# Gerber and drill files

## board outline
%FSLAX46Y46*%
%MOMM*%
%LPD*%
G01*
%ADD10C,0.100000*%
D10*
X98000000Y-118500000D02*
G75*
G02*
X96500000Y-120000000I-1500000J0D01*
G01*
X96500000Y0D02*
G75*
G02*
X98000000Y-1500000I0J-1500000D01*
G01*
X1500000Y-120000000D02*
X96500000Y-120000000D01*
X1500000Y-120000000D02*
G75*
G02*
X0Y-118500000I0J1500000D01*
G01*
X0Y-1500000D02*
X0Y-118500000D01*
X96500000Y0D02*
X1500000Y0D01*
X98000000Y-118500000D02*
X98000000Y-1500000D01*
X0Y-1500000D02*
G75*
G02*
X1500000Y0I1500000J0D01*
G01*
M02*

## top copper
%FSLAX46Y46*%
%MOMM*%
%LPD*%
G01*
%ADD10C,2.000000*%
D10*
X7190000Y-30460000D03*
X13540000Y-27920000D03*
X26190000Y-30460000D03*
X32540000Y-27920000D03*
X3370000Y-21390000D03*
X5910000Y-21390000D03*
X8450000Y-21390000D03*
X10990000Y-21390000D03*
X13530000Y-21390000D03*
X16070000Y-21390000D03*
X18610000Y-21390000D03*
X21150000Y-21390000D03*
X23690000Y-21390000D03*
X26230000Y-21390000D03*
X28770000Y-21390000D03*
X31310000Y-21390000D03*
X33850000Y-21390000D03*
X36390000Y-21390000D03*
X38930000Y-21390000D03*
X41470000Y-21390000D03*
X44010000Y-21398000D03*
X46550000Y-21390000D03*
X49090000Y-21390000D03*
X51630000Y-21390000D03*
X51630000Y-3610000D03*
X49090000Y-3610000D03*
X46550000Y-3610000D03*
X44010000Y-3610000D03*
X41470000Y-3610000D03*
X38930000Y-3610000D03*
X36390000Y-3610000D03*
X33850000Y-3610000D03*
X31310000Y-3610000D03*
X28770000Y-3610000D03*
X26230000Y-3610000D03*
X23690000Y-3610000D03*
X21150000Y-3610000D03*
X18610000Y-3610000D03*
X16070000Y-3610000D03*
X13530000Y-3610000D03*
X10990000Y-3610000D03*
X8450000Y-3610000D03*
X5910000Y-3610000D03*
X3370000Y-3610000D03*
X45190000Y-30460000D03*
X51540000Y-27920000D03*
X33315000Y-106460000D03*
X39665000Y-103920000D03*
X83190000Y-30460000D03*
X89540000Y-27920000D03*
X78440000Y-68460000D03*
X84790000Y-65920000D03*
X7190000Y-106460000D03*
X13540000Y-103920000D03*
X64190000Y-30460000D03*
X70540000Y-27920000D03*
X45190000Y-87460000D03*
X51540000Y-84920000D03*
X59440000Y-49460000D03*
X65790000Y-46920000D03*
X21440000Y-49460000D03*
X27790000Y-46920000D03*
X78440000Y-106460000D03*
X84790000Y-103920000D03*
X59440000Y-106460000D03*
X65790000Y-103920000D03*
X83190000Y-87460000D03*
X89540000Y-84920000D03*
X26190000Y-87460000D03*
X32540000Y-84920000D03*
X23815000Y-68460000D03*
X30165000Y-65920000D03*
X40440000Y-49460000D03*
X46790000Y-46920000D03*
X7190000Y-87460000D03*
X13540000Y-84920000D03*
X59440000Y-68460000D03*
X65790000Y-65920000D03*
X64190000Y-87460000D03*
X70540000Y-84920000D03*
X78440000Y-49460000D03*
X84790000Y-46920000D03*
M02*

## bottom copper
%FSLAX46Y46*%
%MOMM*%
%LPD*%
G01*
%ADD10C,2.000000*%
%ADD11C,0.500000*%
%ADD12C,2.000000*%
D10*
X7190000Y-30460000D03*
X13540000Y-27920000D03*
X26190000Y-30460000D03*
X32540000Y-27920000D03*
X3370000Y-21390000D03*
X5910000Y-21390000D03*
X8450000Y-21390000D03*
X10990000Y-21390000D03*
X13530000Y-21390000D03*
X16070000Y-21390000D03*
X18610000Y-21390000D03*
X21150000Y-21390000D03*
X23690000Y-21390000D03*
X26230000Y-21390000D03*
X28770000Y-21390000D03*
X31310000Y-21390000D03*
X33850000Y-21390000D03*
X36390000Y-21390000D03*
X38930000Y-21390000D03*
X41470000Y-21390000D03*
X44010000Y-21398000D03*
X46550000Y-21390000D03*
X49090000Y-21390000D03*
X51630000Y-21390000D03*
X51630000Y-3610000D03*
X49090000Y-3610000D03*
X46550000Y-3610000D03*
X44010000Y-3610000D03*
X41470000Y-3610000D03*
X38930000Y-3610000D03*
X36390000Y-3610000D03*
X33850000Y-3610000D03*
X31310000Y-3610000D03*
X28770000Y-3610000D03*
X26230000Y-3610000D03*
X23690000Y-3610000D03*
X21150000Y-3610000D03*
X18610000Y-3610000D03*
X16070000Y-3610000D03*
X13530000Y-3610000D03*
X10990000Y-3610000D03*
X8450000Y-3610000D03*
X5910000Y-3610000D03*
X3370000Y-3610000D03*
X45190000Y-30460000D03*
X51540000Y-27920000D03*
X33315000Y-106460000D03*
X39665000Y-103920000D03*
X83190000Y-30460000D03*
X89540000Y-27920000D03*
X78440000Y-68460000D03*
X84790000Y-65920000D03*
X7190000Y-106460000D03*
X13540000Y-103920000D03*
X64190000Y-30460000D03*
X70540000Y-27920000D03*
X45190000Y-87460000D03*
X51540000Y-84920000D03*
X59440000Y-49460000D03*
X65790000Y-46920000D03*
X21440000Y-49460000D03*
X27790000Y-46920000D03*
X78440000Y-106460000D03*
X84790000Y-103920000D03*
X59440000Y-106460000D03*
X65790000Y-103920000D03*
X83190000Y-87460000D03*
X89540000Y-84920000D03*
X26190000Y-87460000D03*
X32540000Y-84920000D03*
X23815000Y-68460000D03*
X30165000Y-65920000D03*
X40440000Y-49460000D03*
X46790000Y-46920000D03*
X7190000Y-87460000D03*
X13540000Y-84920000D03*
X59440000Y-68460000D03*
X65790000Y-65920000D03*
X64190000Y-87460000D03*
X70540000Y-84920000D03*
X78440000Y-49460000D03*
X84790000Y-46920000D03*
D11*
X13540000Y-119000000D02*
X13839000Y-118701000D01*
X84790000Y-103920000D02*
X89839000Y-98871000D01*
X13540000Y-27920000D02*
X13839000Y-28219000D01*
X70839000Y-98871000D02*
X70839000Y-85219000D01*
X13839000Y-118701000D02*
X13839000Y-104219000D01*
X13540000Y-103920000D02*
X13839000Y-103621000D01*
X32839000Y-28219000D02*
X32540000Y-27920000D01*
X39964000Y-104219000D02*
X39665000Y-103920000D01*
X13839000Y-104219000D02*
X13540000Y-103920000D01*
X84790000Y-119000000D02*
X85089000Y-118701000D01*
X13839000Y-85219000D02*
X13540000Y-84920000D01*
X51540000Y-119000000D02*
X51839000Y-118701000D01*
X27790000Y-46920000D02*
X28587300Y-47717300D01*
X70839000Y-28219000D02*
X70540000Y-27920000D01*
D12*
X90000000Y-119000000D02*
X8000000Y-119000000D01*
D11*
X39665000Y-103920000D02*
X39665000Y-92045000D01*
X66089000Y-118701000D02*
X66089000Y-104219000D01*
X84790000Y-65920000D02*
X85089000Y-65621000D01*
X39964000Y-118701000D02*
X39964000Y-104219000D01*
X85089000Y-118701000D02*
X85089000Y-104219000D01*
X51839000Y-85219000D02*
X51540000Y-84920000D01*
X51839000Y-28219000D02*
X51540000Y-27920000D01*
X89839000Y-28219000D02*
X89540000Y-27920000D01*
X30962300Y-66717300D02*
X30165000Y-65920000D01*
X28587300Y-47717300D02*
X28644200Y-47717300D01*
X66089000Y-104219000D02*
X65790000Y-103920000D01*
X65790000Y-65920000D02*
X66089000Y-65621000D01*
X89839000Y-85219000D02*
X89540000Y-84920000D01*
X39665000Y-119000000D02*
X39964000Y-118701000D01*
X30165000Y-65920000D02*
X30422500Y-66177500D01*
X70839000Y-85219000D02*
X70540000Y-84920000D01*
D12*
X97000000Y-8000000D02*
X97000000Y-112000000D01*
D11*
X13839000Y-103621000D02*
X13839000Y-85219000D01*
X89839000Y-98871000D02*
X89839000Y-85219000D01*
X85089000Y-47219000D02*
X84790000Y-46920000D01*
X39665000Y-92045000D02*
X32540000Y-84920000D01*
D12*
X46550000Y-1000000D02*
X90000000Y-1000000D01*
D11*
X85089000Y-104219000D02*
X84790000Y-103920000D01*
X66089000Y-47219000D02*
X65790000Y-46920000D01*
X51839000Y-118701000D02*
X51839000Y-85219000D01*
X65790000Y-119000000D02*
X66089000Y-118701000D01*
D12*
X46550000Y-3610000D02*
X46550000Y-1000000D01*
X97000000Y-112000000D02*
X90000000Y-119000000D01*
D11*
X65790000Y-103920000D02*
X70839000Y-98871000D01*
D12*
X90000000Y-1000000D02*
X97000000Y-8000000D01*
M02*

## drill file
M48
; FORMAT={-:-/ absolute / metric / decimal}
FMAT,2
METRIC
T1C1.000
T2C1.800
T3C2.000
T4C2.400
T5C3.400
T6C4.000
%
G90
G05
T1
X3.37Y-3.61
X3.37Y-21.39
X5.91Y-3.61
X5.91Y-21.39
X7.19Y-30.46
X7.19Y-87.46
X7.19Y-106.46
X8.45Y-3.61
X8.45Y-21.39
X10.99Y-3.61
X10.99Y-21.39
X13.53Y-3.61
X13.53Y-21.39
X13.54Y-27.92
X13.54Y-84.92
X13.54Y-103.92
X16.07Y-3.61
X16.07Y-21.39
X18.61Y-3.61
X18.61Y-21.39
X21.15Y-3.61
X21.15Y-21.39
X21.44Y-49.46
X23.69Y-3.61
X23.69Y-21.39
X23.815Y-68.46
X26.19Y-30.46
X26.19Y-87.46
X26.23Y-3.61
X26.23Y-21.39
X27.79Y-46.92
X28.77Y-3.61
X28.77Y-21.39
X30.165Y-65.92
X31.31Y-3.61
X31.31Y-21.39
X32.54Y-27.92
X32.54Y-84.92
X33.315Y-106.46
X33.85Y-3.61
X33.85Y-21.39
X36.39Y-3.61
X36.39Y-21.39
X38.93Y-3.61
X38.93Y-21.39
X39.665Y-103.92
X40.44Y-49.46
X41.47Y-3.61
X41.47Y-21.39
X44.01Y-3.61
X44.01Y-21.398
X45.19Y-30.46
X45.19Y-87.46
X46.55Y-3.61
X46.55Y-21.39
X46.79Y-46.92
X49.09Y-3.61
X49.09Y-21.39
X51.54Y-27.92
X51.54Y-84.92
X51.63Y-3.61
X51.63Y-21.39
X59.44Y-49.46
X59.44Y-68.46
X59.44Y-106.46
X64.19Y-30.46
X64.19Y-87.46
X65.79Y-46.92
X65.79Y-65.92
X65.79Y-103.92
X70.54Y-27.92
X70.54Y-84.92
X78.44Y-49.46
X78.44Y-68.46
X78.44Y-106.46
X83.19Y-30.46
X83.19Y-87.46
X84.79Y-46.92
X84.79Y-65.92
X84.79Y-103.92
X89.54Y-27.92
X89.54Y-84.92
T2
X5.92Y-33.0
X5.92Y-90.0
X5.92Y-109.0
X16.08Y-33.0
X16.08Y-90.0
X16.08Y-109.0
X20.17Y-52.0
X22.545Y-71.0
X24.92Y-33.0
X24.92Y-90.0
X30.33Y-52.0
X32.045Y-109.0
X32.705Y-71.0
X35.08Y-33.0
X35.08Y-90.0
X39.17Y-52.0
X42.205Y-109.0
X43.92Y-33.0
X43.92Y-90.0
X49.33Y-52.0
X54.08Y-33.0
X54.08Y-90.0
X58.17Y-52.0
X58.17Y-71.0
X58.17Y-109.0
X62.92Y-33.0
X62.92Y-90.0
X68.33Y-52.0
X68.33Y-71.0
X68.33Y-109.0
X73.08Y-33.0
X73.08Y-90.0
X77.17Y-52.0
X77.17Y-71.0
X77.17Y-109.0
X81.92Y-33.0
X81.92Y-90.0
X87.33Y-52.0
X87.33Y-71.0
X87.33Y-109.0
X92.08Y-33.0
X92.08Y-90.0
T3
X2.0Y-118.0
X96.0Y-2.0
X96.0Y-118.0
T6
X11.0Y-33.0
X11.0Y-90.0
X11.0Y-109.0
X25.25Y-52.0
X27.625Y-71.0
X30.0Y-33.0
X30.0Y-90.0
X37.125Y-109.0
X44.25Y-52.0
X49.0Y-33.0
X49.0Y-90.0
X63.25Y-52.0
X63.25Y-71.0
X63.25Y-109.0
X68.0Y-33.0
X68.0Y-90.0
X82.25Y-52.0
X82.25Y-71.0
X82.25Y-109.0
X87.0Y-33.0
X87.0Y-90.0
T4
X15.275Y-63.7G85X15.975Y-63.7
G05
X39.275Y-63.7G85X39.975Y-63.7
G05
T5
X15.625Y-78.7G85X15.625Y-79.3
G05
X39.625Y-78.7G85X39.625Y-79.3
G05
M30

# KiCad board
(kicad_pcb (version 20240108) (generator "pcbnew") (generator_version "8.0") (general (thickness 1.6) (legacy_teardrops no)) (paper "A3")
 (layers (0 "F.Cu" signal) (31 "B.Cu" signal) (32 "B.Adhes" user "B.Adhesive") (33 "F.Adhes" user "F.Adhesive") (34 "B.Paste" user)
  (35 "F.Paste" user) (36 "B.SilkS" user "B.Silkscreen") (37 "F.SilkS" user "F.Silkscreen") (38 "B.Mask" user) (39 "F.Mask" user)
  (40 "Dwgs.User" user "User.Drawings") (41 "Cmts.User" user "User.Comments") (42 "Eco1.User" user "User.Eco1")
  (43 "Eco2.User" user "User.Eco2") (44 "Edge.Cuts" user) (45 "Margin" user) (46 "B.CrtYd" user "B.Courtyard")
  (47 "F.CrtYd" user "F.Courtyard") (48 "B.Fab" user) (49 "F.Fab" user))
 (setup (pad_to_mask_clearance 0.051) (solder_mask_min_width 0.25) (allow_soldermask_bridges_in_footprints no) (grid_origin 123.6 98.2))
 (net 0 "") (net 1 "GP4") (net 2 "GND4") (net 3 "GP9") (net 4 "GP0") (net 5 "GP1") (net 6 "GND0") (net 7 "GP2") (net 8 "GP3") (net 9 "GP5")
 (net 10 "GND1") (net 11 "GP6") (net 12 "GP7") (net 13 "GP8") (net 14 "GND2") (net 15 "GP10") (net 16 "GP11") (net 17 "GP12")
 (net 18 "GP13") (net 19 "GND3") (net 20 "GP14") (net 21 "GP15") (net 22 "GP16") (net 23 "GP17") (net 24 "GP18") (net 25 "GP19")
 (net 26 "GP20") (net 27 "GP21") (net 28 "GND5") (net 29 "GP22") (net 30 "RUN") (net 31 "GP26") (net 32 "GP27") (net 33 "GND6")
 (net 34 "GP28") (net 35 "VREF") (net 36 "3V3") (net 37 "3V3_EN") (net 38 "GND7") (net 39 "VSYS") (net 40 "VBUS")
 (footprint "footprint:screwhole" (layer "F.Cu") (at 96 2)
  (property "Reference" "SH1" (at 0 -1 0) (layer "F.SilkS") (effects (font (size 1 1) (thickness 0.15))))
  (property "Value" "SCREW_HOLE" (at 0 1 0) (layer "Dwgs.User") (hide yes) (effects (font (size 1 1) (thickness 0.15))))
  (pad "" np_thru_hole circle (at 0 0) (size 2 2) (drill 2) (layers "*.Cu" "*.Mask")))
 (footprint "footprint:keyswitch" (layer "F.Cu") (at 11 33)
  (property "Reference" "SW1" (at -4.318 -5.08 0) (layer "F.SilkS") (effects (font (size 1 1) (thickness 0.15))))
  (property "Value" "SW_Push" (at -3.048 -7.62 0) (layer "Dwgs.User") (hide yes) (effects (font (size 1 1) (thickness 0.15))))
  (pad "" np_thru_hole circle (at -5.08 0) (size 1.8 1.8) (drill 1.8) (layers "*.Cu" "*.Mask"))
  (pad "" np_thru_hole circle (at 0 0) (size 4 4) (drill 4) (layers "*.Cu" "*.Mask"))
  (pad "" np_thru_hole circle (at 5.08 0) (size 1.8 1.8) (drill 1.8) (layers "*.Cu" "*.Mask"))
  (pad "1" thru_hole circle (at -3.81 -2.54) (size 2 2) (drill 1) (layers "*.Cu" "*.Mask") (remove_unused_layers no) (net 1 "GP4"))
  (pad "2" thru_hole circle (at 2.54 -5.08) (size 2 2) (drill 1) (layers "*.Cu" "*.Mask") (remove_unused_layers no) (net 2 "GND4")))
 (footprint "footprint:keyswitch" (layer "F.Cu") (at 30 33)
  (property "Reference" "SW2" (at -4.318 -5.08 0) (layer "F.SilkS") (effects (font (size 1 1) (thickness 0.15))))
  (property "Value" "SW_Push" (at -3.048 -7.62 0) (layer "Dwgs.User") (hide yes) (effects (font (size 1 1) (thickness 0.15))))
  (pad "" np_thru_hole circle (at -5.08 0) (size 1.8 1.8) (drill 1.8) (layers "*.Cu" "*.Mask"))
  (pad "" np_thru_hole circle (at 0 0) (size 4 4) (drill 4) (layers "*.Cu" "*.Mask"))
  (pad "" np_thru_hole circle (at 5.08 0) (size 1.8 1.8) (drill 1.8) (layers "*.Cu" "*.Mask"))
  (pad "1" thru_hole circle (at -3.81 -2.54) (size 2 2) (drill 1) (layers "*.Cu" "*.Mask") (remove_unused_layers no) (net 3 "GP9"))
  (pad "2" thru_hole circle (at 2.54 -5.08) (size 2 2) (drill 1) (layers "*.Cu" "*.Mask") (remove_unused_layers no) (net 2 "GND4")))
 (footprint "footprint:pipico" (layer "F.Cu") (at 27.5 12.5)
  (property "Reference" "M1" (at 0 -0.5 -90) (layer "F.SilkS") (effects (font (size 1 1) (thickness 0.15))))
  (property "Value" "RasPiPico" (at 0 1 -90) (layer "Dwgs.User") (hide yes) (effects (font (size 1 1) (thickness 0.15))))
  (pad "1" thru_hole circle (at -24.13 8.89 270) (size 2 2) (drill 1) (layers "*.Cu" "*.Mask") (remove_unused_layers no) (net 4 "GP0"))
  (pad "2" thru_hole circle (at -21.59 8.89 270) (size 2 2) (drill 1) (layers "*.Cu" "*.Mask") (remove_unused_layers no) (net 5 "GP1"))
  (pad "3" thru_hole circle (at -19.05 8.89 270) (size 2 2) (drill 1) (layers "*.Cu" "*.Mask") (remove_unused_layers no) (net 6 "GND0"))
  (pad "4" thru_hole circle (at -16.51 8.89 270) (size 2 2) (drill 1) (layers "*.Cu" "*.Mask") (remove_unused_layers no) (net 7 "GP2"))
  (pad "5" thru_hole circle (at -13.97 8.89 270) (size 2 2) (drill 1) (layers "*.Cu" "*.Mask") (remove_unused_layers no) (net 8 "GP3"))
  (pad "6" thru_hole circle (at -11.43 8.89 270) (size 2 2) (drill 1) (layers "*.Cu" "*.Mask") (remove_unused_layers no) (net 1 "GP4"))
  (pad "7" thru_hole circle (at -8.89 8.89 270) (size 2 2) (drill 1) (layers "*.Cu" "*.Mask") (remove_unused_layers no) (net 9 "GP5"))
  (pad "8" thru_hole circle (at -6.35 8.89 270) (size 2 2) (drill 1) (layers "*.Cu" "*.Mask") (remove_unused_layers no) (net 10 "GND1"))
  (pad "9" thru_hole circle (at -3.81 8.89 270) (size 2 2) (drill 1) (layers "*.Cu" "*.Mask") (remove_unused_layers no) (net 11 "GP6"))
  (pad "10" thru_hole circle (at -1.27 8.89 270) (size 2 2) (drill 1) (layers "*.Cu" "*.Mask") (remove_unused_layers no) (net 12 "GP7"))
  (pad "11" thru_hole circle (at 1.27 8.89 270) (size 2 2) (drill 1) (layers "*.Cu" "*.Mask") (remove_unused_layers no) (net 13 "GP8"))
  (pad "12" thru_hole circle (at 3.81 8.89 270) (size 2 2) (drill 1) (layers "*.Cu" "*.Mask") (remove_unused_layers no) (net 3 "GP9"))
  (pad "13" thru_hole circle (at 6.35 8.89 270) (size 2 2) (drill 1) (layers "*.Cu" "*.Mask") (remove_unused_layers no) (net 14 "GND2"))
  (pad "14" thru_hole circle (at 8.89 8.89 270) (size 2 2) (drill 1) (layers "*.Cu" "*.Mask") (remove_unused_layers no) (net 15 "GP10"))
  (pad "15" thru_hole circle (at 11.43 8.89 270) (size 2 2) (drill 1) (layers "*.Cu" "*.Mask") (remove_unused_layers no) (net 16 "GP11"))
  (pad "16" thru_hole circle (at 13.97 8.89 270) (size 2 2) (drill 1) (layers "*.Cu" "*.Mask") (remove_unused_layers no) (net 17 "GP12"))
  (pad "17" thru_hole circle (at 16.51 8.898 270) (size 2 2) (drill 1) (layers "*.Cu" "*.Mask") (remove_unused_layers no) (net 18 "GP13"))
  (pad "18" thru_hole circle (at 19.05 8.89 270) (size 2 2) (drill 1) (layers "*.Cu" "*.Mask") (remove_unused_layers no) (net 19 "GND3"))
  (pad "19" thru_hole circle (at 21.59 8.89 270) (size 2 2) (drill 1) (layers "*.Cu" "*.Mask") (remove_unused_layers no) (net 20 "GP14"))
  (pad "20" thru_hole circle (at 24.13 8.89 270) (size 2 2) (drill 1) (layers "*.Cu" "*.Mask") (remove_unused_layers no) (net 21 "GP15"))
  (pad "21" thru_hole circle (at 24.13 -8.89 270) (size 2 2) (drill 1) (layers "*.Cu" "*.Mask") (remove_unused_layers no) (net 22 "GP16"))
  (pad "22" thru_hole circle (at 21.59 -8.89 270) (size 2 2) (drill 1) (layers "*.Cu" "*.Mask") (remove_unused_layers no) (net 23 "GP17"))
  (pad "23" thru_hole circle (at 19.05 -8.89 270) (size 2 2) (drill 1) (layers "*.Cu" "*.Mask") (remove_unused_layers no) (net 2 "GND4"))
  (pad "24" thru_hole circle (at 16.51 -8.89 270) (size 2 2) (drill 1) (layers "*.Cu" "*.Mask") (remove_unused_layers no) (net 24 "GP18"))
  (pad "25" thru_hole circle (at 13.97 -8.89 270) (size 2 2) (drill 1) (layers "*.Cu" "*.Mask") (remove_unused_layers no) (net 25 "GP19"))
  (pad "26" thru_hole circle (at 11.43 -8.89 270) (size 2 2) (drill 1) (layers "*.Cu" "*.Mask") (remove_unused_layers no) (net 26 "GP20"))
  (pad "27" thru_hole circle (at 8.89 -8.89 270) (size 2 2) (drill 1) (layers "*.Cu" "*.Mask") (remove_unused_layers no) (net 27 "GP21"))
  (pad "28" thru_hole circle (at 6.35 -8.89 270) (size 2 2) (drill 1) (layers "*.Cu" "*.Mask") (remove_unused_layers no) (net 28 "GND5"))
  (pad "29" thru_hole circle (at 3.81 -8.89 270) (size 2 2) (drill 1) (layers "*.Cu" "*.Mask") (remove_unused_layers no) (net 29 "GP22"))
  (pad "30" thru_hole circle (at 1.27 -8.89 270) (size 2 2) (drill 1) (layers "*.Cu" "*.Mask") (remove_unused_layers no) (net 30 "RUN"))
  (pad "31" thru_hole circle (at -1.27 -8.89 270) (size 2 2) (drill 1) (layers "*.Cu" "*.Mask") (remove_unused_layers no) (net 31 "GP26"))
  (pad "32" thru_hole circle (at -3.81 -8.89 270) (size 2 2) (drill 1) (layers "*.Cu" "*.Mask") (remove_unused_layers no) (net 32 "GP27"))
  (pad "33" thru_hole circle (at -6.35 -8.89 270) (size 2 2) (drill 1) (layers "*.Cu" "*.Mask") (remove_unused_layers no) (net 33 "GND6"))
  (pad "34" thru_hole circle (at -8.89 -8.89 270) (size 2 2) (drill 1) (layers "*.Cu" "*.Mask") (remove_unused_layers no) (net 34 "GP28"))
  (pad "35" thru_hole circle (at -11.43 -8.89 270) (size 2 2) (drill 1) (layers "*.Cu" "*.Mask") (remove_unused_layers no) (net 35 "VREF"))
  (pad "36" thru_hole circle (at -13.97 -8.89 270) (size 2 2) (drill 1) (layers "*.Cu" "*.Mask") (remove_unused_layers no) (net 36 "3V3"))
  (pad "37" thru_hole circle (at -16.51 -8.89 270) (size 2 2) (drill 1) (layers "*.Cu" "*.Mask") (remove_unused_layers no) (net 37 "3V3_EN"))
  (pad "38" thru_hole circle (at -19.05 -8.89 270) (size 2 2) (drill 1) (layers "*.Cu" "*.Mask") (remove_unused_layers no) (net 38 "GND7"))
  (pad "39" thru_hole circle (at -21.59 -8.89 270) (size 2 2) (drill 1) (layers "*.Cu" "*.Mask") (remove_unused_layers no) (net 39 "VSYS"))
  (pad "40" thru_hole circle (at -24.13 -8.89 270) (size 2 2) (drill 1) (layers "*.Cu" "*.Mask") (remove_unused_layers no) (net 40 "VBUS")))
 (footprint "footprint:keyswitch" (layer "F.Cu") (at 49 33)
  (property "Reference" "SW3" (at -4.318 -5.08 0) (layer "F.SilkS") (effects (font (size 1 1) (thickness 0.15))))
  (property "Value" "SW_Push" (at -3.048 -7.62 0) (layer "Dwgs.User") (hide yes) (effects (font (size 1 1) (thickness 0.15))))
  (pad "" np_thru_hole circle (at -5.08 0) (size 1.8 1.8) (drill 1.8) (layers "*.Cu" "*.Mask"))
  (pad "" np_thru_hole circle (at 0 0) (size 4 4) (drill 4) (layers "*.Cu" "*.Mask"))
  (pad "" np_thru_hole circle (at 5.08 0) (size 1.8 1.8) (drill 1.8) (layers "*.Cu" "*.Mask"))
  (pad "1" thru_hole circle (at -3.81 -2.54) (size 2 2) (drill 1) (layers "*.Cu" "*.Mask") (remove_unused_layers no) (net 20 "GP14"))
  (pad "2" thru_hole circle (at 2.54 -5.08) (size 2 2) (drill 1) (layers "*.Cu" "*.Mask") (remove_unused_layers no) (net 2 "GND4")))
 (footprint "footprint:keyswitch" (layer "F.Cu") (at 37.125 109)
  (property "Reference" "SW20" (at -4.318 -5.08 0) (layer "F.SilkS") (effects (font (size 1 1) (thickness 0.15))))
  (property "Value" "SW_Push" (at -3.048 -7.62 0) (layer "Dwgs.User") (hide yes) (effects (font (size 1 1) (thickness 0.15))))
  (pad "" np_thru_hole circle (at -5.08 0) (size 1.8 1.8) (drill 1.8) (layers "*.Cu" "*.Mask"))
  (pad "" np_thru_hole circle (at 0 0) (size 4 4) (drill 4) (layers "*.Cu" "*.Mask"))
  (pad "" np_thru_hole circle (at 5.08 0) (size 1.8 1.8) (drill 1.8) (layers "*.Cu" "*.Mask"))
  (pad "1" thru_hole circle (at -3.81 -2.54) (size 2 2) (drill 1) (layers "*.Cu" "*.Mask") (remove_unused_layers no) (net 9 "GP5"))
  (pad "2" thru_hole circle (at 2.54 -5.08) (size 2 2) (drill 1) (layers "*.Cu" "*.Mask") (remove_unused_layers no) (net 2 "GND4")))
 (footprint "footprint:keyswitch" (layer "F.Cu") (at 87 33)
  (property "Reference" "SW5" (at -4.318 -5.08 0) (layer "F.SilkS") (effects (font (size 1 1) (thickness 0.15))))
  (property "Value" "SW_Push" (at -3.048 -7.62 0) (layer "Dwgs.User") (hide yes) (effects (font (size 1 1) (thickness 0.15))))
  (pad "" np_thru_hole circle (at -5.08 0) (size 1.8 1.8) (drill 1.8) (layers "*.Cu" "*.Mask"))
  (pad "" np_thru_hole circle (at 0 0) (size 4 4) (drill 4) (layers "*.Cu" "*.Mask"))
  (pad "" np_thru_hole circle (at 5.08 0) (size 1.8 1.8) (drill 1.8) (layers "*.Cu" "*.Mask"))
  (pad "1" thru_hole circle (at -3.81 -2.54) (size 2 2) (drill 1) (layers "*.Cu" "*.Mask") (remove_unused_layers no) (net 22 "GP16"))
  (pad "2" thru_hole circle (at 2.54 -5.08) (size 2 2) (drill 1) (layers "*.Cu" "*.Mask") (remove_unused_layers no) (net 2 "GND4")))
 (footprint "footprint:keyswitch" (layer "F.Cu") (at 82.25 71)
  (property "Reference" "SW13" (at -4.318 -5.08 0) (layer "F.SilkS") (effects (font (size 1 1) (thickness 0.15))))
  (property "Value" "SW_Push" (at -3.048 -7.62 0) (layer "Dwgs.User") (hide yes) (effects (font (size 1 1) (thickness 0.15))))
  (pad "" np_thru_hole circle (at -5.08 0) (size 1.8 1.8) (drill 1.8) (layers "*.Cu" "*.Mask"))
  (pad "" np_thru_hole circle (at 0 0) (size 4 4) (drill 4) (layers "*.Cu" "*.Mask"))
  (pad "" np_thru_hole circle (at 5.08 0) (size 1.8 1.8) (drill 1.8) (layers "*.Cu" "*.Mask"))
  (pad "1" thru_hole circle (at -3.81 -2.54) (size 2 2) (drill 1) (layers "*.Cu" "*.Mask") (remove_unused_layers no) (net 24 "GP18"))
  (pad "2" thru_hole circle (at 2.54 -5.08) (size 2 2) (drill 1) (layers "*.Cu" "*.Mask") (remove_unused_layers no) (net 2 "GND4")))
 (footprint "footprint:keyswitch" (layer "F.Cu") (at 11 109)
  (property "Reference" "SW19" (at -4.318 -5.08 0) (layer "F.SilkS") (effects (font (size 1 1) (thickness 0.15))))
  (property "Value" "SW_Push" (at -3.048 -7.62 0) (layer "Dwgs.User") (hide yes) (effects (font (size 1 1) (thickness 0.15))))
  (pad "" np_thru_hole circle (at -5.08 0) (size 1.8 1.8) (drill 1.8) (layers "*.Cu" "*.Mask"))
  (pad "" np_thru_hole circle (at 0 0) (size 4 4) (drill 4) (layers "*.Cu" "*.Mask"))
  (pad "" np_thru_hole circle (at 5.08 0) (size 1.8 1.8) (drill 1.8) (layers "*.Cu" "*.Mask"))
  (pad "1" thru_hole circle (at -3.81 -2.54) (size 2 2) (drill 1) (layers "*.Cu" "*.Mask") (remove_unused_layers no) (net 4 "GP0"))
  (pad "2" thru_hole circle (at 2.54 -5.08) (size 2 2) (drill 1) (layers "*.Cu" "*.Mask") (remove_unused_layers no) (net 2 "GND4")))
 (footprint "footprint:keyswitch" (layer "F.Cu") (at 68 33)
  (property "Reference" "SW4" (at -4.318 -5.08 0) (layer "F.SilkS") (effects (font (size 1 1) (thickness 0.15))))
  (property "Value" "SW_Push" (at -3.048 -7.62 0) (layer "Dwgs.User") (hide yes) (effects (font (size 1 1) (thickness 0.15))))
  (pad "" np_thru_hole circle (at -5.08 0) (size 1.8 1.8) (drill 1.8) (layers "*.Cu" "*.Mask"))
  (pad "" np_thru_hole circle (at 0 0) (size 4 4) (drill 4) (layers "*.Cu" "*.Mask"))
  (pad "" np_thru_hole circle (at 5.08 0) (size 1.8 1.8) (drill 1.8) (layers "*.Cu" "*.Mask"))
  (pad "1" thru_hole circle (at -3.81 -2.54) (size 2 2) (drill 1) (layers "*.Cu" "*.Mask") (remove_unused_layers no) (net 27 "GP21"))
  (pad "2" thru_hole circle (at 2.54 -5.08) (size 2 2) (drill 1) (layers "*.Cu" "*.Mask") (remove_unused_layers no) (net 2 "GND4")))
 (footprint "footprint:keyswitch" (layer "F.Cu") (at 49 90)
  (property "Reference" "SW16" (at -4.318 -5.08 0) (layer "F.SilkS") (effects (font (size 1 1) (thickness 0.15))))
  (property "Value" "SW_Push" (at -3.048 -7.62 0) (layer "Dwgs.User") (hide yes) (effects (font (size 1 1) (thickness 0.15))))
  (pad "" np_thru_hole circle (at -5.08 0) (size 1.8 1.8) (drill 1.8) (layers "*.Cu" "*.Mask"))
  (pad "" np_thru_hole circle (at 0 0) (size 4 4) (drill 4) (layers "*.Cu" "*.Mask"))
  (pad "" np_thru_hole circle (at 5.08 0) (size 1.8 1.8) (drill 1.8) (layers "*.Cu" "*.Mask"))
  (pad "1" thru_hole circle (at -3.81 -2.54) (size 2 2) (drill 1) (layers "*.Cu" "*.Mask") (remove_unused_layers no) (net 16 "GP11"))
  (pad "2" thru_hole circle (at 2.54 -5.08) (size 2 2) (drill 1) (layers "*.Cu" "*.Mask") (remove_unused_layers no) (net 2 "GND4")))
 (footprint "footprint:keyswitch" (layer "F.Cu") (at 63.25 52)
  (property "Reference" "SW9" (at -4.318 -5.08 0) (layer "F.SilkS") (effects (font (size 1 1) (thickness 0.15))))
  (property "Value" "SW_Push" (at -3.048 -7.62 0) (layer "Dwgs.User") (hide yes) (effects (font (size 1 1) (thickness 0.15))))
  (pad "" np_thru_hole circle (at -5.08 0) (size 1.8 1.8) (drill 1.8) (layers "*.Cu" "*.Mask"))
  (pad "" np_thru_hole circle (at 0 0) (size 4 4) (drill 4) (layers "*.Cu" "*.Mask"))
  (pad "" np_thru_hole circle (at 5.08 0) (size 1.8 1.8) (drill 1.8) (layers "*.Cu" "*.Mask"))
  (pad "1" thru_hole circle (at -3.81 -2.54) (size 2 2) (drill 1) (layers "*.Cu" "*.Mask") (remove_unused_layers no) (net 29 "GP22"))
  (pad "2" thru_hole circle (at 2.54 -5.08) (size 2 2) (drill 1) (layers "*.Cu" "*.Mask") (remove_unused_layers no) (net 2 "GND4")))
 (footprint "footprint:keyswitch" (layer "F.Cu") (at 25.25 52)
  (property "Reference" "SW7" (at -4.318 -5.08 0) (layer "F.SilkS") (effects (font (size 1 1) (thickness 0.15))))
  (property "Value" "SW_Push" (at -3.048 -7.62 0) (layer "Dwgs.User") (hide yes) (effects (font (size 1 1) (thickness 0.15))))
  (pad "" np_thru_hole circle (at -5.08 0) (size 1.8 1.8) (drill 1.8) (layers "*.Cu" "*.Mask"))
  (pad "" np_thru_hole circle (at 0 0) (size 4 4) (drill 4) (layers "*.Cu" "*.Mask"))
  (pad "" np_thru_hole circle (at 5.08 0) (size 1.8 1.8) (drill 1.8) (layers "*.Cu" "*.Mask"))
  (pad "1" thru_hole circle (at -3.81 -2.54) (size 2 2) (drill 1) (layers "*.Cu" "*.Mask") (remove_unused_layers no) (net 13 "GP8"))
  (pad "2" thru_hole circle (at 2.54 -5.08) (size 2 2) (drill 1) (layers "*.Cu" "*.Mask") (remove_unused_layers no) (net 2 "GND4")))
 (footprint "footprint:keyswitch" (layer "F.Cu") (at 82.25 109)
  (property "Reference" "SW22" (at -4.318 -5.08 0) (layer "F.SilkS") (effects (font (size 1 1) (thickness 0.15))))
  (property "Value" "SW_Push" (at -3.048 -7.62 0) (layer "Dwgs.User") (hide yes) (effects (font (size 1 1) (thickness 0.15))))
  (pad "" np_thru_hole circle (at -5.08 0) (size 1.8 1.8) (drill 1.8) (layers "*.Cu" "*.Mask"))
  (pad "" np_thru_hole circle (at 0 0) (size 4 4) (drill 4) (layers "*.Cu" "*.Mask"))
  (pad "" np_thru_hole circle (at 5.08 0) (size 1.8 1.8) (drill 1.8) (layers "*.Cu" "*.Mask"))
  (pad "1" thru_hole circle (at -3.81 -2.54) (size 2 2) (drill 1) (layers "*.Cu" "*.Mask") (remove_unused_layers no) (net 26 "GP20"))
  (pad "2" thru_hole circle (at 2.54 -5.08) (size 2 2) (drill 1) (layers "*.Cu" "*.Mask") (remove_unused_layers no) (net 2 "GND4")))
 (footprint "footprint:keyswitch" (layer "F.Cu") (at 63.25 109)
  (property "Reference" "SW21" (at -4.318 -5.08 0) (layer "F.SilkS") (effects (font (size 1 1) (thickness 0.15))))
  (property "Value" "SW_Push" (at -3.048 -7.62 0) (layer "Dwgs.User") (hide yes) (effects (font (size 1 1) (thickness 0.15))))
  (pad "" np_thru_hole circle (at -5.08 0) (size 1.8 1.8) (drill 1.8) (layers "*.Cu" "*.Mask"))
  (pad "" np_thru_hole circle (at 0 0) (size 4 4) (drill 4) (layers "*.Cu" "*.Mask"))
  (pad "" np_thru_hole circle (at 5.08 0) (size 1.8 1.8) (drill 1.8) (layers "*.Cu" "*.Mask"))
  (pad "1" thru_hole circle (at -3.81 -2.54) (size 2 2) (drill 1) (layers "*.Cu" "*.Mask") (remove_unused_layers no) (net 34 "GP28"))
  (pad "2" thru_hole circle (at 2.54 -5.08) (size 2 2) (drill 1) (layers "*.Cu" "*.Mask") (remove_unused_layers no) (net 2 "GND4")))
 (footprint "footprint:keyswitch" (layer "F.Cu") (at 87 90)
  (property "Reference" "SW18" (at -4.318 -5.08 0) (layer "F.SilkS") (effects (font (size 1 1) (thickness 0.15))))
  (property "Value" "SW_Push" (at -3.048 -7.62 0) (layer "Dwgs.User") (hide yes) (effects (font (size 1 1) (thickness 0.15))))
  (pad "" np_thru_hole circle (at -5.08 0) (size 1.8 1.8) (drill 1.8) (layers "*.Cu" "*.Mask"))
  (pad "" np_thru_hole circle (at 0 0) (size 4 4) (drill 4) (layers "*.Cu" "*.Mask"))
  (pad "" np_thru_hole circle (at 5.08 0) (size 1.8 1.8) (drill 1.8) (layers "*.Cu" "*.Mask"))
  (pad "1" thru_hole circle (at -3.81 -2.54) (size 2 2) (drill 1) (layers "*.Cu" "*.Mask") (remove_unused_layers no) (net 25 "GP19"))
  (pad "2" thru_hole circle (at 2.54 -5.08) (size 2 2) (drill 1) (layers "*.Cu" "*.Mask") (remove_unused_layers no) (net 2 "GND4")))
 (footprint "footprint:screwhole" (layer "F.Cu") (at 2 118)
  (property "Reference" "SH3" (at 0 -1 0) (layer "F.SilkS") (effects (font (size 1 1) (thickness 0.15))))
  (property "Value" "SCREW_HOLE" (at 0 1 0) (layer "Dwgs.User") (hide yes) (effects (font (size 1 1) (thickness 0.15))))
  (pad "" np_thru_hole circle (at 0 0) (size 2 2) (drill 2) (layers "*.Cu" "*.Mask")))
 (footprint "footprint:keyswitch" (layer "F.Cu") (at 30 90)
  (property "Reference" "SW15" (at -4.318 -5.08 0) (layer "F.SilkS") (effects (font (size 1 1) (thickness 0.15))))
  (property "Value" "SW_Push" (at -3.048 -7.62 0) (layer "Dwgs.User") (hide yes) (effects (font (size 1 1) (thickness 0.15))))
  (pad "" np_thru_hole circle (at -5.08 0) (size 1.8 1.8) (drill 1.8) (layers "*.Cu" "*.Mask"))
  (pad "" np_thru_hole circle (at 0 0) (size 4 4) (drill 4) (layers "*.Cu" "*.Mask"))
  (pad "" np_thru_hole circle (at 5.08 0) (size 1.8 1.8) (drill 1.8) (layers "*.Cu" "*.Mask"))
  (pad "1" thru_hole circle (at -3.81 -2.54) (size 2 2) (drill 1) (layers "*.Cu" "*.Mask") (remove_unused_layers no) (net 11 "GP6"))
  (pad "2" thru_hole circle (at 2.54 -5.08) (size 2 2) (drill 1) (layers "*.Cu" "*.Mask") (remove_unused_layers no) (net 2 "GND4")))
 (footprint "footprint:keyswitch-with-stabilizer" (layer "F.Cu") (at 27.625 71)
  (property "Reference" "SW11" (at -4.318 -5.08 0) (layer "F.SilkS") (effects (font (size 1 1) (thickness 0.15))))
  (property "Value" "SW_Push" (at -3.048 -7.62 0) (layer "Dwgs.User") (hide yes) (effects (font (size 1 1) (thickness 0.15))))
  (pad "" np_thru_hole oval (at -12 -7.3) (size 3.1 2.4) (drill oval 3.1 2.4) (layers "*.Cu" "*.Mask"))
  (pad "" np_thru_hole oval (at -12 8) (size 3.4 4) (drill oval 3.4 4) (layers "*.Cu" "*.Mask"))
  (pad "" np_thru_hole circle (at -5.08 0) (size 1.8 1.8) (drill 1.8) (layers "*.Cu" "*.Mask"))
  (pad "" np_thru_hole circle (at 0 0) (size 4 4) (drill 4) (layers "*.Cu" "*.Mask"))
  (pad "" np_thru_hole circle (at 5.08 0) (size 1.8 1.8) (drill 1.8) (layers "*.Cu" "*.Mask"))
  (pad "" np_thru_hole oval (at 12 -7.3) (size 3.1 2.4) (drill oval 3.1 2.4) (layers "*.Cu" "*.Mask"))
  (pad "" np_thru_hole oval (at 12 8) (size 3.4 4) (drill oval 3.4 4) (layers "*.Cu" "*.Mask"))
  (pad "1" thru_hole circle (at -3.81 -2.54) (size 2 2) (drill 1) (layers "*.Cu" "*.Mask") (remove_unused_layers no) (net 12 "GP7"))
  (pad "2" thru_hole circle (at 2.54 -5.08) (size 2 2) (drill 1) (layers "*.Cu" "*.Mask") (remove_unused_layers no) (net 2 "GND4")))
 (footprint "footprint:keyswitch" (layer "F.Cu") (at 44.25 52)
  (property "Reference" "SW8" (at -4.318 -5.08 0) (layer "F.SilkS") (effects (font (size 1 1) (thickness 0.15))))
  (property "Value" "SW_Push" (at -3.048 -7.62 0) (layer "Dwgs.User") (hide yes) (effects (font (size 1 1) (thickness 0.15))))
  (pad "" np_thru_hole circle (at -5.08 0) (size 1.8 1.8) (drill 1.8) (layers "*.Cu" "*.Mask"))
  (pad "" np_thru_hole circle (at 0 0) (size 4 4) (drill 4) (layers "*.Cu" "*.Mask"))
  (pad "" np_thru_hole circle (at 5.08 0) (size 1.8 1.8) (drill 1.8) (layers "*.Cu" "*.Mask"))
  (pad "1" thru_hole circle (at -3.81 -2.54) (size 2 2) (drill 1) (layers "*.Cu" "*.Mask") (remove_unused_layers no) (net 18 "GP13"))
  (pad "2" thru_hole circle (at 2.54 -5.08) (size 2 2) (drill 1) (layers "*.Cu" "*.Mask") (remove_unused_layers no) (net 2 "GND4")))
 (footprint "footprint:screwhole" (layer "F.Cu") (at 96 118)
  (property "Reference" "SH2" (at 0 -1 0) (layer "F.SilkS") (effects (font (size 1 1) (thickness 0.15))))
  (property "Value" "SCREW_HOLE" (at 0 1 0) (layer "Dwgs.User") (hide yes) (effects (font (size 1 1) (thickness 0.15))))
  (pad "" np_thru_hole circle (at 0 0) (size 2 2) (drill 2) (layers "*.Cu" "*.Mask")))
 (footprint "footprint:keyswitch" (layer "F.Cu") (at 11 90)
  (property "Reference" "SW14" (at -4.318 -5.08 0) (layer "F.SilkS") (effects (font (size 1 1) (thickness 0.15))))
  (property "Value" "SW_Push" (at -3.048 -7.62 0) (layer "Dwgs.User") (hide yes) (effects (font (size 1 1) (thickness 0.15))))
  (pad "" np_thru_hole circle (at -5.08 0) (size 1.8 1.8) (drill 1.8) (layers "*.Cu" "*.Mask"))
  (pad "" np_thru_hole circle (at 0 0) (size 4 4) (drill 4) (layers "*.Cu" "*.Mask"))
  (pad "" np_thru_hole circle (at 5.08 0) (size 1.8 1.8) (drill 1.8) (layers "*.Cu" "*.Mask"))
  (pad "1" thru_hole circle (at -3.81 -2.54) (size 2 2) (drill 1) (layers "*.Cu" "*.Mask") (remove_unused_layers no) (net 5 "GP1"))
  (pad "2" thru_hole circle (at 2.54 -5.08) (size 2 2) (drill 1) (layers "*.Cu" "*.Mask") (remove_unused_layers no) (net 2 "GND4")))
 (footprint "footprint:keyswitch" (layer "F.Cu") (at 63.25 71)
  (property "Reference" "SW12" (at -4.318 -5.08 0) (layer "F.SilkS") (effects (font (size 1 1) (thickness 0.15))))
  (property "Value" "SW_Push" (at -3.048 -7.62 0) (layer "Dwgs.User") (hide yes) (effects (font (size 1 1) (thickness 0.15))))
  (pad "" np_thru_hole circle (at -5.08 0) (size 1.8 1.8) (drill 1.8) (layers "*.Cu" "*.Mask"))
  (pad "" np_thru_hole circle (at 0 0) (size 4 4) (drill 4) (layers "*.Cu" "*.Mask"))
  (pad "" np_thru_hole circle (at 5.08 0) (size 1.8 1.8) (drill 1.8) (layers "*.Cu" "*.Mask"))
  (pad "1" thru_hole circle (at -3.81 -2.54) (size 2 2) (drill 1) (layers "*.Cu" "*.Mask") (remove_unused_layers no) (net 31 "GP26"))
  (pad "2" thru_hole circle (at 2.54 -5.08) (size 2 2) (drill 1) (layers "*.Cu" "*.Mask") (remove_unused_layers no) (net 2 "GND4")))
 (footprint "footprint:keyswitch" (layer "F.Cu") (at 68 90)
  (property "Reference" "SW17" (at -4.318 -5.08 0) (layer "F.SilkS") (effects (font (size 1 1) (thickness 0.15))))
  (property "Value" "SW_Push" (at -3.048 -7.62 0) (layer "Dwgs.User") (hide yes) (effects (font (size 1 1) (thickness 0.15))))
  (pad "" np_thru_hole circle (at -5.08 0) (size 1.8 1.8) (drill 1.8) (layers "*.Cu" "*.Mask"))
  (pad "" np_thru_hole circle (at 0 0) (size 4 4) (drill 4) (layers "*.Cu" "*.Mask"))
  (pad "" np_thru_hole circle (at 5.08 0) (size 1.8 1.8) (drill 1.8) (layers "*.Cu" "*.Mask"))
  (pad "1" thru_hole circle (at -3.81 -2.54) (size 2 2) (drill 1) (layers "*.Cu" "*.Mask") (remove_unused_layers no) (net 32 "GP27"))
  (pad "2" thru_hole circle (at 2.54 -5.08) (size 2 2) (drill 1) (layers "*.Cu" "*.Mask") (remove_unused_layers no) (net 2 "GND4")))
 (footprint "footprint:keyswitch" (layer "F.Cu") (at 82.25 52)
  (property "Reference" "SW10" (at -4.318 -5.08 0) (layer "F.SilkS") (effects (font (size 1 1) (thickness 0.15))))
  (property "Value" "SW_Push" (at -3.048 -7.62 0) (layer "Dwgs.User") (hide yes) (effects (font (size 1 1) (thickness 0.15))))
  (pad "" np_thru_hole circle (at -5.08 0) (size 1.8 1.8) (drill 1.8) (layers "*.Cu" "*.Mask"))
  (pad "" np_thru_hole circle (at 0 0) (size 4 4) (drill 4) (layers "*.Cu" "*.Mask"))
  (pad "" np_thru_hole circle (at 5.08 0) (size 1.8 1.8) (drill 1.8) (layers "*.Cu" "*.Mask"))
  (pad "1" thru_hole circle (at -3.81 -2.54) (size 2 2) (drill 1) (layers "*.Cu" "*.Mask") (remove_unused_layers no) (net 23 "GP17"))
  (pad "2" thru_hole circle (at 2.54 -5.08) (size 2 2) (drill 1) (layers "*.Cu" "*.Mask") (remove_unused_layers no) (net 2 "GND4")))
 (gr_arc (start 98 118.5) (mid 97.56066 119.56066) (end 96.5 120) (stroke (width 0.1) (type solid)) (layer "Edge.Cuts"))
 (gr_arc (start 96.5 0) (mid 97.56066 0.43934) (end 98 1.5) (stroke (width 0.1) (type solid)) (layer "Edge.Cuts"))
 (gr_line (start 1.5 120) (end 96.5 120) (stroke (width 0.1) (type solid)) (layer "Edge.Cuts"))
 (gr_arc (start 1.5 120) (mid 0.43934 119.56066) (end 0 118.5) (stroke (width 0.1) (type solid)) (layer "Edge.Cuts"))
 (gr_line (start 0 1.5) (end 0 118.5) (stroke (width 0.1) (type solid)) (layer "Edge.Cuts"))
 (gr_line (start 96.5 0) (end 1.5 0) (stroke (width 0.1) (type solid)) (layer "Edge.Cuts"))
 (gr_line (start 98 118.5) (end 98 1.5) (stroke (width 0.1) (type solid)) (layer "Edge.Cuts"))
 (gr_arc (start 0 1.5) (mid 0.43934 0.43934) (end 1.5 0) (stroke (width 0.1) (type solid)) (layer "Edge.Cuts"))
 (segment (start 13.54 119) (end 13.839 118.701) (width 0.5) (layer "B.Cu") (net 2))
 (segment (start 84.79 103.92) (end 89.839 98.871) (width 0.5) (layer "B.Cu") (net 2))
 (segment (start 13.54 27.92) (end 13.839 28.219) (width 0.5) (layer "B.Cu") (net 2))
 (segment (start 70.839 98.871) (end 70.839 85.219) (width 0.5) (layer "B.Cu") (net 2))
 (segment (start 13.839 118.701) (end 13.839 104.219) (width 0.5) (layer "B.Cu") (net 2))
 (segment (start 13.54 103.92) (end 13.839 103.621) (width 0.5) (layer "B.Cu") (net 2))
 (segment (start 32.839 28.219) (end 32.54 27.92) (width 0.5) (layer "B.Cu") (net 2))
 (segment (start 39.964 104.219) (end 39.665 103.92) (width 0.5) (layer "B.Cu") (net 2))
 (segment (start 13.839 104.219) (end 13.54 103.92) (width 0.5) (layer "B.Cu") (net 2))
 (segment (start 84.79 119) (end 85.089 118.701) (width 0.5) (layer "B.Cu") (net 2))
 (segment (start 13.839 85.219) (end 13.54 84.92) (width 0.5) (layer "B.Cu") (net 2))
 (segment (start 51.54 119) (end 51.839 118.701) (width 0.5) (layer "B.Cu") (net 2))
 (segment (start 27.79 46.92) (end 28.5873 47.7173) (width 0.5) (layer "B.Cu") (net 2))
 (segment (start 70.839 28.219) (end 70.54 27.92) (width 0.5) (layer "B.Cu") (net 2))
 (segment (start 90 119) (end 8 119) (width 2) (layer "B.Cu") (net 2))
 (segment (start 39.665 103.92) (end 39.665 92.045) (width 0.5) (layer "B.Cu") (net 2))
 (segment (start 66.089 118.701) (end 66.089 104.219) (width 0.5) (layer "B.Cu") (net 2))
 (segment (start 84.79 65.92) (end 85.089 65.621) (width 0.5) (layer "B.Cu") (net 2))
 (segment (start 39.964 118.701) (end 39.964 104.219) (width 0.5) (layer "B.Cu") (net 2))
 (segment (start 85.089 118.701) (end 85.089 104.219) (width 0.5) (layer "B.Cu") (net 2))
 (segment (start 51.839 85.219) (end 51.54 84.92) (width 0.5) (layer "B.Cu") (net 2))
 (segment (start 51.839 28.219) (end 51.54 27.92) (width 0.5) (layer "B.Cu") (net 2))
 (segment (start 89.839 28.219) (end 89.54 27.92) (width 0.5) (layer "B.Cu") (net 2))
 (segment (start 30.9623 66.7173) (end 30.165 65.92) (width 0.5) (layer "B.Cu") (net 2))
 (segment (start 28.5873 47.7173) (end 28.6442 47.7173) (width 0.5) (layer "B.Cu") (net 2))
 (segment (start 66.089 104.219) (end 65.79 103.92) (width 0.5) (layer "B.Cu") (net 2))
 (segment (start 65.79 65.92) (end 66.089 65.621) (width 0.5) (layer "B.Cu") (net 2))
 (segment (start 89.839 85.219) (end 89.54 84.92) (width 0.5) (layer "B.Cu") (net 2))
 (segment (start 39.665 119) (end 39.964 118.701) (width 0.5) (layer "B.Cu") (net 2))
 (segment (start 30.165 65.92) (end 30.4225 66.1775) (width 0.5) (layer "B.Cu") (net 2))
 (segment (start 70.839 85.219) (end 70.54 84.92) (width 0.5) (layer "B.Cu") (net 2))
 (segment (start 97 8) (end 97 112) (width 2) (layer "B.Cu") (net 2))
 (segment (start 13.839 103.621) (end 13.839 85.219) (width 0.5) (layer "B.Cu") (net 2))
 (segment (start 89.839 98.871) (end 89.839 85.219) (width 0.5) (layer "B.Cu") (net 2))
 (segment (start 85.089 47.219) (end 84.79 46.92) (width 0.5) (layer "B.Cu") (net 2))
 (segment (start 39.665 92.045) (end 32.54 84.92) (width 0.5) (layer "B.Cu") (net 2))
 (segment (start 46.55 1) (end 90 1) (width 2) (layer "B.Cu") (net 2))
 (segment (start 85.089 104.219) (end 84.79 103.92) (width 0.5) (layer "B.Cu") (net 2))
 (segment (start 66.089 47.219) (end 65.79 46.92) (width 0.5) (layer "B.Cu") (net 2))
 (segment (start 51.839 118.701) (end 51.839 85.219) (width 0.5) (layer "B.Cu") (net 2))
 (segment (start 65.79 119) (end 66.089 118.701) (width 0.5) (layer "B.Cu") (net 2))
 (segment (start 46.55 3.61) (end 46.55 1) (width 2) (layer "B.Cu") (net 2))
 (segment (start 97 112) (end 90 119) (width 2) (layer "B.Cu") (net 2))
 (segment (start 65.79 103.92) (end 70.839 98.871) (width 0.5) (layer "B.Cu") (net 2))
 (segment (start 90 1) (end 97 8) (width 2) (layer "B.Cu") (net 2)))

